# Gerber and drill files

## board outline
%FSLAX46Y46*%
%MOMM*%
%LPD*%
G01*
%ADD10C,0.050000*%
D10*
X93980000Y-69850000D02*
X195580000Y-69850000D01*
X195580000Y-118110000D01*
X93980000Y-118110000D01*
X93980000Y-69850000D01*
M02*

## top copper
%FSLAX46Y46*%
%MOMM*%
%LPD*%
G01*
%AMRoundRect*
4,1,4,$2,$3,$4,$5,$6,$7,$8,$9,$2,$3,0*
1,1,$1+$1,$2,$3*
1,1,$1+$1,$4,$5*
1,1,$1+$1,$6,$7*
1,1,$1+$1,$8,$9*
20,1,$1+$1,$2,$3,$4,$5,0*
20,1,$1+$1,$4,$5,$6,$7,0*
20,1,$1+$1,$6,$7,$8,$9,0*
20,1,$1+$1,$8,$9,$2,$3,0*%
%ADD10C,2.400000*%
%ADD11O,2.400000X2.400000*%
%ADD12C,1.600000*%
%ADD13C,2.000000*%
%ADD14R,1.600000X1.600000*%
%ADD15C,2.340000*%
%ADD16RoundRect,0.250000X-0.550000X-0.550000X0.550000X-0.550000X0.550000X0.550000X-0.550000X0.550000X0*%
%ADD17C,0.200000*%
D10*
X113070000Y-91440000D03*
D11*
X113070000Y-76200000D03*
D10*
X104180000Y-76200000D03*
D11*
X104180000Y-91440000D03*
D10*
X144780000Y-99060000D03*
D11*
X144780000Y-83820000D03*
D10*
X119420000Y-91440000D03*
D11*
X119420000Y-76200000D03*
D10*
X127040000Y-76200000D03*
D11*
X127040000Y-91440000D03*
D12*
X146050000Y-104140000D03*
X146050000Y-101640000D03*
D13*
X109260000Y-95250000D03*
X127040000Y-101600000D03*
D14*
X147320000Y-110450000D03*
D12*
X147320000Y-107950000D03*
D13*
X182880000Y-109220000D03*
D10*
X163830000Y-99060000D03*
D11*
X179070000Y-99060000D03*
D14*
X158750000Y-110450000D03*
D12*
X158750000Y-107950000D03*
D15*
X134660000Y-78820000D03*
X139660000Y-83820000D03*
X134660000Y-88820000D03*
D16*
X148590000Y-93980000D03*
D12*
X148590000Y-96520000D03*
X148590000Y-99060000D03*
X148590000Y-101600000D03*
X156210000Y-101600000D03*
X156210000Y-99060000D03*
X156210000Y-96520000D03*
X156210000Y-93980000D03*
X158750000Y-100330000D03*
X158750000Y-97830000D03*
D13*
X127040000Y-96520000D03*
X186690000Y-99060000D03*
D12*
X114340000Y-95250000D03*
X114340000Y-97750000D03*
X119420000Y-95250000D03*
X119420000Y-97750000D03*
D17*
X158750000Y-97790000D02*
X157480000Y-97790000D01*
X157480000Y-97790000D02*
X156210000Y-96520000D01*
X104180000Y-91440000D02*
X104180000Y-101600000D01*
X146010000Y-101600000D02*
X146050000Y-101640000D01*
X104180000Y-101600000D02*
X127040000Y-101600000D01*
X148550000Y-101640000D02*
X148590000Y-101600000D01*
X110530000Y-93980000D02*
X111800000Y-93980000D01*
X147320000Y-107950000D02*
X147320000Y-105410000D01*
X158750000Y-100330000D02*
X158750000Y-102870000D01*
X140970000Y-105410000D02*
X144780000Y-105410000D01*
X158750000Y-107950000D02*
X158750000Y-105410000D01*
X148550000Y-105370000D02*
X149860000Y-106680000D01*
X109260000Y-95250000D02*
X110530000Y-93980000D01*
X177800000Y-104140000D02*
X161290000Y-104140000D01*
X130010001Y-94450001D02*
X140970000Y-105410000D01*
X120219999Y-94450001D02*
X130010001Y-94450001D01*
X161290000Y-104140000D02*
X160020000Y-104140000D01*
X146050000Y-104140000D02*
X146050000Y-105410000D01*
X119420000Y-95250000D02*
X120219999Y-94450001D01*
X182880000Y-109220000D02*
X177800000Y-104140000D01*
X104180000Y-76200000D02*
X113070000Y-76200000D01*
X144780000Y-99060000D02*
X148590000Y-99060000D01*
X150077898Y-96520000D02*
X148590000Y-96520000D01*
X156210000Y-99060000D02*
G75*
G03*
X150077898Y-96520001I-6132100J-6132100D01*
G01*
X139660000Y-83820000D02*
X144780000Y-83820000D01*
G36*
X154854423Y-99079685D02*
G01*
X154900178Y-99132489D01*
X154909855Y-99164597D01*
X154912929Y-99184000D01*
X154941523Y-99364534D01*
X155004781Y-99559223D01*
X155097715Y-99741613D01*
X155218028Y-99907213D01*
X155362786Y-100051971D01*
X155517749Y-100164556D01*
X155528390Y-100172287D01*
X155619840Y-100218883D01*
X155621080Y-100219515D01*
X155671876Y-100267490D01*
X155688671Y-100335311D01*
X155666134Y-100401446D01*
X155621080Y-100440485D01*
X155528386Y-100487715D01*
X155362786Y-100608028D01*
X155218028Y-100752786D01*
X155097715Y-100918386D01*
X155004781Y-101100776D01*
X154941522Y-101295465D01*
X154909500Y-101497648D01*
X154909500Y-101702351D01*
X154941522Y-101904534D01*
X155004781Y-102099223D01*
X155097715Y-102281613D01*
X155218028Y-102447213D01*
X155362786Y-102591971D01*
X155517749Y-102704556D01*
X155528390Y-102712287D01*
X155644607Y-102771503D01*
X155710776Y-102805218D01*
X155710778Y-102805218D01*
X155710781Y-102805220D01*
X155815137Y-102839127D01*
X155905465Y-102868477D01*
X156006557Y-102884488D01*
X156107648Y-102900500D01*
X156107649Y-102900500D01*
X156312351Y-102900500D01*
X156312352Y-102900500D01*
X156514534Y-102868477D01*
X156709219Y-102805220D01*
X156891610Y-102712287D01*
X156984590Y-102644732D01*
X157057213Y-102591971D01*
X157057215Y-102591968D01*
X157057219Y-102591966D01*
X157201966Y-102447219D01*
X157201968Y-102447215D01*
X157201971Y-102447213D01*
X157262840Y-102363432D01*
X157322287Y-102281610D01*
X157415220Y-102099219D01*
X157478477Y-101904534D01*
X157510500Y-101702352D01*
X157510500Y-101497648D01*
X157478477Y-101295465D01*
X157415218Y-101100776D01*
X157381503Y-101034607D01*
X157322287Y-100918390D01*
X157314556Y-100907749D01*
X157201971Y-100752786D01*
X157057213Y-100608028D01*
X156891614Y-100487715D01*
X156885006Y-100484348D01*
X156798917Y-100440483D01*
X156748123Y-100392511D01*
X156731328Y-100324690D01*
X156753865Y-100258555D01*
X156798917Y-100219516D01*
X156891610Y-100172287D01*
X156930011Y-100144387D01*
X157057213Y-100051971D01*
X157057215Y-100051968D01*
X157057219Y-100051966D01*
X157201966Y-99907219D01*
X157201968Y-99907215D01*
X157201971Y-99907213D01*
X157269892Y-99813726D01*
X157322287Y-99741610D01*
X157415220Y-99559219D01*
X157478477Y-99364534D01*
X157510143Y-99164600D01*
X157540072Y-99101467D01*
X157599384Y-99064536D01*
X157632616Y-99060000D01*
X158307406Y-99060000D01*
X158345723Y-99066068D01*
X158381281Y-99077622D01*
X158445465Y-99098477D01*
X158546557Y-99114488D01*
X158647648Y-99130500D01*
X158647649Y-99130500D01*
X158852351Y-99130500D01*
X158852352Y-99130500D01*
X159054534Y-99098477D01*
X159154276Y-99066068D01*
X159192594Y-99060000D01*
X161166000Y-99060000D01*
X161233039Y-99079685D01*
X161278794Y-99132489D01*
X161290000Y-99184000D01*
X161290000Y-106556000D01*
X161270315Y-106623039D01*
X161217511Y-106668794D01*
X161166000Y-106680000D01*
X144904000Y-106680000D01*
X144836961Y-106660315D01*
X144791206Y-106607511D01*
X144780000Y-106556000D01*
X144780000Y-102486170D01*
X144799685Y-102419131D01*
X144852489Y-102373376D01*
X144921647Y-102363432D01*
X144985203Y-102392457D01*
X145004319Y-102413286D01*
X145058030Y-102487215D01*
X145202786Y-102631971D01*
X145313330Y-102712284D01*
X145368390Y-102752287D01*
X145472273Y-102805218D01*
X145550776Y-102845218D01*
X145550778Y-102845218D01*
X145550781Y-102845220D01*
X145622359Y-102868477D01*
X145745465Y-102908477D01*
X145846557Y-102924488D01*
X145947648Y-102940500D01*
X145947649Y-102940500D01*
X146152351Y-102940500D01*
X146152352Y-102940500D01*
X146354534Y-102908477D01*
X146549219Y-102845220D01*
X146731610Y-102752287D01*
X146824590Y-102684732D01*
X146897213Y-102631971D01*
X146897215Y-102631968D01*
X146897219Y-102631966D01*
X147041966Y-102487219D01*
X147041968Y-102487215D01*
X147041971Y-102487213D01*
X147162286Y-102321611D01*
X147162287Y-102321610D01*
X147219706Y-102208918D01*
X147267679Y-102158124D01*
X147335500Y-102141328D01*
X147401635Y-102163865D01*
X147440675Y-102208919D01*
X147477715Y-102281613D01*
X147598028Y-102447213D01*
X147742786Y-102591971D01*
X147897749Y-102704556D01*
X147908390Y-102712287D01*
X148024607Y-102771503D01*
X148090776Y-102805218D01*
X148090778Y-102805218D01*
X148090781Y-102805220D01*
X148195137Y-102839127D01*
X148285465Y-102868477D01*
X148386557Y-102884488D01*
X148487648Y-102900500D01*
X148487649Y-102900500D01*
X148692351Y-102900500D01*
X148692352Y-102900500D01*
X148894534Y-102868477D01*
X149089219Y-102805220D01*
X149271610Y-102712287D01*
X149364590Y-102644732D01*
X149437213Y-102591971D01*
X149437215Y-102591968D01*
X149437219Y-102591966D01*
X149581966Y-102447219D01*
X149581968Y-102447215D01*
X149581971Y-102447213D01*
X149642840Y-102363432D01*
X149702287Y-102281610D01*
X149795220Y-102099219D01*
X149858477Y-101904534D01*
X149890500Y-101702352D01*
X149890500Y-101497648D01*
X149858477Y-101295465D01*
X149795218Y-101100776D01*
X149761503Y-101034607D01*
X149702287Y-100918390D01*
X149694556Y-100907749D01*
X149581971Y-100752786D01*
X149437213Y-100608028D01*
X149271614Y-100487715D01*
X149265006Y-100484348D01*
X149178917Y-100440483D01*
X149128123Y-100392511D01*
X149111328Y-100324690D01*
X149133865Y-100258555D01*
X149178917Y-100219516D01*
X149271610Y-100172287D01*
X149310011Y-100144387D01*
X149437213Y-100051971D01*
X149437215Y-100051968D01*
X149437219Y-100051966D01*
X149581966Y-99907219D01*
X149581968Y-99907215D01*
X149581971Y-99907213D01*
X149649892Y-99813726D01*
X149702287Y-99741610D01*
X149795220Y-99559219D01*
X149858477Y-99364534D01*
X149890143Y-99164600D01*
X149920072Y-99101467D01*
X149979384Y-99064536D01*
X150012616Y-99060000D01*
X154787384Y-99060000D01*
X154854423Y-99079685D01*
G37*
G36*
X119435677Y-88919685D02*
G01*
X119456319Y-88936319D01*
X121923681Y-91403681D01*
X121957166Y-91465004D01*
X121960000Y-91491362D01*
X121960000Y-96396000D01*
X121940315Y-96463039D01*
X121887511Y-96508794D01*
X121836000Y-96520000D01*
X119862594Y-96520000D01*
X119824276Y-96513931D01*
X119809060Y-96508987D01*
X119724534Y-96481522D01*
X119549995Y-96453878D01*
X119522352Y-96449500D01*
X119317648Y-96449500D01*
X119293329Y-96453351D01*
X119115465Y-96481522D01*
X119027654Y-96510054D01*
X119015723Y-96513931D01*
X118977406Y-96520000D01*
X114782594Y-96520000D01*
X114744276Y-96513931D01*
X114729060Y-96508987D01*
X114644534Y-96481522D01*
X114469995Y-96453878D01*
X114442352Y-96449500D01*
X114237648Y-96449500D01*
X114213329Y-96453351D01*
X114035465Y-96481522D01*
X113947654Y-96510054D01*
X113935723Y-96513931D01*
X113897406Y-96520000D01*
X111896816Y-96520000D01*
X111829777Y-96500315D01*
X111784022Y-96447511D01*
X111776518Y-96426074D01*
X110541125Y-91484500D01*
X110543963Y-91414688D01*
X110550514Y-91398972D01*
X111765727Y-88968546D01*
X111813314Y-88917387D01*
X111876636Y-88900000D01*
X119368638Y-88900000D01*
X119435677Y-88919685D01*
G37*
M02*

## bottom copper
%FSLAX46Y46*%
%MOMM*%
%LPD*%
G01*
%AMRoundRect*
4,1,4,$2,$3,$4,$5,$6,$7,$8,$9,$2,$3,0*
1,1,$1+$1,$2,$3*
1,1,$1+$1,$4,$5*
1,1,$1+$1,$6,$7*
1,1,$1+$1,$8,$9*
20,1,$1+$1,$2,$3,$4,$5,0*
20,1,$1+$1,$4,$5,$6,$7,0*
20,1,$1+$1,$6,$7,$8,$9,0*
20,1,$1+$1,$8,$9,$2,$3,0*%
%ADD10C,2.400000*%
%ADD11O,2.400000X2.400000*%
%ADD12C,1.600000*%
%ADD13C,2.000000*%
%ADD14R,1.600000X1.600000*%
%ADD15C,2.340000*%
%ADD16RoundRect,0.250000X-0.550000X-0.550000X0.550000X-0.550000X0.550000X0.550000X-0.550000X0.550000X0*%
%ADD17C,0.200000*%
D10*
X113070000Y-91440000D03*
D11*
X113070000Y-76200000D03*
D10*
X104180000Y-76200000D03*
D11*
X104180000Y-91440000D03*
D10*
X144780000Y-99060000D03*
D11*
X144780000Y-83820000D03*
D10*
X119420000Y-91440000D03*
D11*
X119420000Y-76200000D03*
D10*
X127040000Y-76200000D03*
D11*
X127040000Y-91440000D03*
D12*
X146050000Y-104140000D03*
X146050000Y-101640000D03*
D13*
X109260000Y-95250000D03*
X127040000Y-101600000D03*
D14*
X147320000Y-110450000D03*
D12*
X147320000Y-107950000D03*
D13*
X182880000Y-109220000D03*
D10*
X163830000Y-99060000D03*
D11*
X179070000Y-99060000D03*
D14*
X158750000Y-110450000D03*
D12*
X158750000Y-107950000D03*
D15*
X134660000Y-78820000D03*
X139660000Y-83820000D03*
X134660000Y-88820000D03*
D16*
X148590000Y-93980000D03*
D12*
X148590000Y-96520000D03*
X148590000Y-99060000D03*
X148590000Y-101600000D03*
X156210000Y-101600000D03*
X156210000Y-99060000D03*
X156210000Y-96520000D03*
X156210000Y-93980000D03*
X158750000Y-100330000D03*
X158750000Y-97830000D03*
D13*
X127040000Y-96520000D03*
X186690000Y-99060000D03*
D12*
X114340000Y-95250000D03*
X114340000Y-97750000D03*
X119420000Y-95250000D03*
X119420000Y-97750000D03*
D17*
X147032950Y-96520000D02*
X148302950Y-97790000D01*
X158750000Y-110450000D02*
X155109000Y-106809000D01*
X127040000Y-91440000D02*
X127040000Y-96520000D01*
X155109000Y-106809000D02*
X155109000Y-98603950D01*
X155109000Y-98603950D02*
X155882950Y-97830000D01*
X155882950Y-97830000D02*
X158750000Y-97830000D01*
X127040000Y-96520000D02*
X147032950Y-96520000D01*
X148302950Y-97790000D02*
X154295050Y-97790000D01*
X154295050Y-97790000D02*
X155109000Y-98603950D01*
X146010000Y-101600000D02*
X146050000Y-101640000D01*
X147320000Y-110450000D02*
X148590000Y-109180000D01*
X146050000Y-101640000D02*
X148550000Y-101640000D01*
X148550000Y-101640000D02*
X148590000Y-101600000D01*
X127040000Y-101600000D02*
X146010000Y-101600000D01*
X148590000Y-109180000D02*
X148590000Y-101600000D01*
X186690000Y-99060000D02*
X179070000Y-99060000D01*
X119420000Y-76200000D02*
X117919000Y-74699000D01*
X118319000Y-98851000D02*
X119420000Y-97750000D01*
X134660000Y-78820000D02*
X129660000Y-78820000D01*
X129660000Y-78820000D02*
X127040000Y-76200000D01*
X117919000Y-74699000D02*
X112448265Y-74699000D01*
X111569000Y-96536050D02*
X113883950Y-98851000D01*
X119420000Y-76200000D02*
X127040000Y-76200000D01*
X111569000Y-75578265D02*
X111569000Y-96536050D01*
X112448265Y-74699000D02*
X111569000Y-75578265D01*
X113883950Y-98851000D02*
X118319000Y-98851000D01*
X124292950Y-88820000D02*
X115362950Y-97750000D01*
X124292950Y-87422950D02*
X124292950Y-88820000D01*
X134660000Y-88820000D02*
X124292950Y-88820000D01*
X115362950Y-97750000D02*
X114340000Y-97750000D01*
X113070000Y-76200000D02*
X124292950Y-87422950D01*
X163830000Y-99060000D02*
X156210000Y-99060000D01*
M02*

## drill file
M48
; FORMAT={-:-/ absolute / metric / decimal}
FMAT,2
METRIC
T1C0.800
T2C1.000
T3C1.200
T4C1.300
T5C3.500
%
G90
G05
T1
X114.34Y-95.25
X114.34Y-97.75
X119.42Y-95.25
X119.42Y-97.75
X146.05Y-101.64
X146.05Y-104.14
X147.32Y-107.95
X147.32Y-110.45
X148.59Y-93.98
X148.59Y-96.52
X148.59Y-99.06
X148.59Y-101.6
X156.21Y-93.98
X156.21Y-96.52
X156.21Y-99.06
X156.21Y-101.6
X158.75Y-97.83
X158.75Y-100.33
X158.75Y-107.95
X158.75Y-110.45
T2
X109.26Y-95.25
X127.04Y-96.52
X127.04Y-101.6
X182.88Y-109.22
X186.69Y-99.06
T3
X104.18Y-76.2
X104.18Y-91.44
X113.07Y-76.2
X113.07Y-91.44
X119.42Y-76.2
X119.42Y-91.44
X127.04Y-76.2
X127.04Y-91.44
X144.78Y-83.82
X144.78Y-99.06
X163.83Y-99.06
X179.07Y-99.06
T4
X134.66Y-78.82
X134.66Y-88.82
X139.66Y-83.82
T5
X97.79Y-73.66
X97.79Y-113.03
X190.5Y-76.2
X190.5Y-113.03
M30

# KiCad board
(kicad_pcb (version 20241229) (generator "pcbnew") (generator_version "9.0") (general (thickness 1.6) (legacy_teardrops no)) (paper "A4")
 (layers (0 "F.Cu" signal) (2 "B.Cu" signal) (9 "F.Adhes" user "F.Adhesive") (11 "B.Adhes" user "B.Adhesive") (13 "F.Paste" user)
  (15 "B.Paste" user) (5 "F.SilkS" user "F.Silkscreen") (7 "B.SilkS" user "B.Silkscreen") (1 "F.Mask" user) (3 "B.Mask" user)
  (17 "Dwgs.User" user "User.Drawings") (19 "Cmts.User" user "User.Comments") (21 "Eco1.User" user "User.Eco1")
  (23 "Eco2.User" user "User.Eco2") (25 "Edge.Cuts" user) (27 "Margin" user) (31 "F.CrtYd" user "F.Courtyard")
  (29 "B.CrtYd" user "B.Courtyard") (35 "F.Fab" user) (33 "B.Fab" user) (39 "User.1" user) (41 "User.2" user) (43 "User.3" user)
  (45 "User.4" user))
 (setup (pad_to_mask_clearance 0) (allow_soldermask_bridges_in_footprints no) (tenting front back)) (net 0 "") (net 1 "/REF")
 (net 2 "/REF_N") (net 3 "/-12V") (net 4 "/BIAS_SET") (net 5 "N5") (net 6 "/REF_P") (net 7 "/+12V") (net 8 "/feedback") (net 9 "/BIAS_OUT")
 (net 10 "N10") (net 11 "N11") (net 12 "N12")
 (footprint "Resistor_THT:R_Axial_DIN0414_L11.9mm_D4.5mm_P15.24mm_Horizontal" (layer "F.Cu") (at 113.07 91.44 90)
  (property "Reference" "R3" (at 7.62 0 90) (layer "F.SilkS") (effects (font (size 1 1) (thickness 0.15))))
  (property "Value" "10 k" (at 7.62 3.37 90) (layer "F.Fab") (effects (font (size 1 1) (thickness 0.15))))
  (pad "1" thru_hole circle (at 0 0 90) (size 2.4 2.4) (drill 1.2) (layers "*.Cu" "*.Mask") (remove_unused_layers no) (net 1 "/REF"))
  (pad "2" thru_hole oval (at 15.24 0 90) (size 2.4 2.4) (drill 1.2) (layers "*.Cu" "*.Mask") (remove_unused_layers no) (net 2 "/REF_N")))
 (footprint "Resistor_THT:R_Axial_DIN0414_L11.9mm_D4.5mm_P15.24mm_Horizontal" (layer "F.Cu") (at 104.18 76.2 -90)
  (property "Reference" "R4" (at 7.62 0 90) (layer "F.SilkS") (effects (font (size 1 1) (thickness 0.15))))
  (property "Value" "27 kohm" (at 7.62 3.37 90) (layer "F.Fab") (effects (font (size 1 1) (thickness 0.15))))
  (pad "1" thru_hole circle (at 0 0 270) (size 2.4 2.4) (drill 1.2) (layers "*.Cu" "*.Mask") (remove_unused_layers no) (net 2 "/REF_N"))
  (pad "2" thru_hole oval (at 15.24 0 270) (size 2.4 2.4) (drill 1.2) (layers "*.Cu" "*.Mask") (remove_unused_layers no) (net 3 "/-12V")))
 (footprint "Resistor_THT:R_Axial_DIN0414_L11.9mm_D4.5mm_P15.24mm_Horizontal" (layer "F.Cu") (at 144.78 99.06 90)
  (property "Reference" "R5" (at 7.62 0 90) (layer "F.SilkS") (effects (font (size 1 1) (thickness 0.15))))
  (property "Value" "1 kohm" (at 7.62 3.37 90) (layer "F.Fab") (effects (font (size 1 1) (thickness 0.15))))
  (pad "1" thru_hole circle (at 0 0 90) (size 2.4 2.4) (drill 1.2) (layers "*.Cu" "*.Mask") (remove_unused_layers no) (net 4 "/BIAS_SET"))
  (pad "2" thru_hole oval (at 15.24 0 90) (size 2.4 2.4) (drill 1.2) (layers "*.Cu" "*.Mask") (remove_unused_layers no) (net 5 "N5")))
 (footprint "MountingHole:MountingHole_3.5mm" (layer "F.Cu") (at 190.5 113.03)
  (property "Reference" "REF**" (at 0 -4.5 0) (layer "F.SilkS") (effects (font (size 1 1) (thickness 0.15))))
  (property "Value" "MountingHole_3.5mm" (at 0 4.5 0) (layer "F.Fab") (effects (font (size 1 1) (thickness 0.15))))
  (pad "" np_thru_hole circle (at 0 0) (size 3.5 3.5) (drill 3.5) (layers "*.Cu" "*.Mask")))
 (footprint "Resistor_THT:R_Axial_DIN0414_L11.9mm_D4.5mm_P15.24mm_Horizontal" (layer "F.Cu") (at 119.42 91.44 90)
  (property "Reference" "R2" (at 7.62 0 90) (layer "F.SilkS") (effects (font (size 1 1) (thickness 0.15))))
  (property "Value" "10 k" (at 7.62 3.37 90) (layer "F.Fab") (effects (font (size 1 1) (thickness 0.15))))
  (pad "1" thru_hole circle (at 0 0 90) (size 2.4 2.4) (drill 1.2) (layers "*.Cu" "*.Mask") (remove_unused_layers no) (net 1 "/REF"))
  (pad "2" thru_hole oval (at 15.24 0 90) (size 2.4 2.4) (drill 1.2) (layers "*.Cu" "*.Mask") (remove_unused_layers no) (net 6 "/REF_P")))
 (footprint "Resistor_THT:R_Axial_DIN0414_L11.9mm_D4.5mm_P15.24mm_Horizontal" (layer "F.Cu") (at 127.04 76.2 -90)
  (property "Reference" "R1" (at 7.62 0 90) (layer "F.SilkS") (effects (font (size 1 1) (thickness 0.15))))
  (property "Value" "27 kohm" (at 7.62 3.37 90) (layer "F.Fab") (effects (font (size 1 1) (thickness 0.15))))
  (pad "1" thru_hole circle (at 0 0 270) (size 2.4 2.4) (drill 1.2) (layers "*.Cu" "*.Mask") (remove_unused_layers no) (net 6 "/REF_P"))
  (pad "2" thru_hole oval (at 15.24 0 270) (size 2.4 2.4) (drill 1.2) (layers "*.Cu" "*.Mask") (remove_unused_layers no) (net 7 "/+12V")))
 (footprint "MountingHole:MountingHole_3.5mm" (layer "F.Cu") (at 190.5 76.2)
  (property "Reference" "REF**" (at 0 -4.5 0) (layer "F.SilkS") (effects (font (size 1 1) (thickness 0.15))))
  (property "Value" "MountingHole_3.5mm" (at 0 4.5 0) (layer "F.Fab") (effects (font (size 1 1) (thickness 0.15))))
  (pad "" np_thru_hole circle (at 0 0) (size 3.5 3.5) (drill 3.5) (layers "*.Cu" "*.Mask")))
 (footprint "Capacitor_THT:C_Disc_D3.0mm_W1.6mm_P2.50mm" (layer "F.Cu") (at 146.05 104.14 90)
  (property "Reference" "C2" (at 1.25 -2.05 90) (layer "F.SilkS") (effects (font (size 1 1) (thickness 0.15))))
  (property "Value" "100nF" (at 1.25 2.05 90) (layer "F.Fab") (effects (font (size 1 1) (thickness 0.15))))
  (pad "1" thru_hole circle (at 0 0 90) (size 1.6 1.6) (drill 0.8) (layers "*.Cu" "*.Mask") (remove_unused_layers no) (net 1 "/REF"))
  (pad "2" thru_hole circle (at 2.5 0 90) (size 1.6 1.6) (drill 0.8) (layers "*.Cu" "*.Mask") (remove_unused_layers no) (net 3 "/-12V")))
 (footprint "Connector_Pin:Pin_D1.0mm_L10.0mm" (layer "F.Cu") (at 109.26 95.25)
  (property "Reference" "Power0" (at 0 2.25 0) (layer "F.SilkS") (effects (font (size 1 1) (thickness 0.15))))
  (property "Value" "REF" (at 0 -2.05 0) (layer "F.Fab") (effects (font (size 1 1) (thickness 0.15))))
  (pad "1" thru_hole circle (at 0 0) (size 2 2) (drill 1) (layers "*.Cu" "*.Mask") (remove_unused_layers no) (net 1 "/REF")))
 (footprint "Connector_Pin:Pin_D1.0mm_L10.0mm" (layer "F.Cu") (at 127.04 101.6)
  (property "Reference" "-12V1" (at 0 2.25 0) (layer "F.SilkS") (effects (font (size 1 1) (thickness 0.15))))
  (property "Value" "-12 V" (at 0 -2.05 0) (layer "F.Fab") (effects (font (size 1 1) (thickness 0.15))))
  (pad "1" thru_hole circle (at 0 0) (size 2 2) (drill 1) (layers "*.Cu" "*.Mask") (remove_unused_layers no) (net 3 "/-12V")))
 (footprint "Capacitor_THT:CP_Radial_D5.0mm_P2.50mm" (layer "F.Cu") (at 147.32 110.45 90)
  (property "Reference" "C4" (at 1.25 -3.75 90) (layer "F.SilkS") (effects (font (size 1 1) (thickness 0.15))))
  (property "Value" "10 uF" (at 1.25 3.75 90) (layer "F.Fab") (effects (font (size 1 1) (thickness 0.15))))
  (pad "1" thru_hole rect (at 0 0 90) (size 1.6 1.6) (drill 0.8) (layers "*.Cu" "*.Mask") (remove_unused_layers no) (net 3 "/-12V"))
  (pad "2" thru_hole circle (at 2.5 0 90) (size 1.6 1.6) (drill 0.8) (layers "*.Cu" "*.Mask") (remove_unused_layers no) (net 1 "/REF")))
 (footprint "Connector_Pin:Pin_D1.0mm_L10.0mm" (layer "F.Cu") (at 182.88 109.22)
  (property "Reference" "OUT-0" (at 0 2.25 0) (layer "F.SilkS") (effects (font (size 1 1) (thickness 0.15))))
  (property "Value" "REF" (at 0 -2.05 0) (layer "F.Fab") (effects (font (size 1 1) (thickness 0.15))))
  (pad "1" thru_hole circle (at 0 0) (size 2 2) (drill 1) (layers "*.Cu" "*.Mask") (remove_unused_layers no) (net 1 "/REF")))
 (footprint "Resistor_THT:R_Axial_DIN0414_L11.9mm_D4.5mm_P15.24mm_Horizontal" (layer "F.Cu") (at 163.83 99.06)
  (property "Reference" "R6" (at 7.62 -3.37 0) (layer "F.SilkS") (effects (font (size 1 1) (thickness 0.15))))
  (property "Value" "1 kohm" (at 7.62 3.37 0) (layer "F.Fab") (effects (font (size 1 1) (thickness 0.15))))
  (pad "1" thru_hole circle (at 0 0) (size 2.4 2.4) (drill 1.2) (layers "*.Cu" "*.Mask") (remove_unused_layers no) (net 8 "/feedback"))
  (pad "2" thru_hole oval (at 15.24 0) (size 2.4 2.4) (drill 1.2) (layers "*.Cu" "*.Mask") (remove_unused_layers no) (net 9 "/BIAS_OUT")))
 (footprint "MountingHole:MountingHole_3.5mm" (layer "F.Cu") (at 97.79 73.66)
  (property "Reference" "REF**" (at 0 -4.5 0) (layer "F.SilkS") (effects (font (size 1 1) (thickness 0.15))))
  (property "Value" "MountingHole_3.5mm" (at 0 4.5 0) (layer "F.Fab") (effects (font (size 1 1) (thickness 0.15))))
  (pad "" np_thru_hole circle (at 0 0) (size 3.5 3.5) (drill 3.5) (layers "*.Cu" "*.Mask")))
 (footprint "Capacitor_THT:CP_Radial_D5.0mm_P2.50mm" (layer "F.Cu") (at 158.75 110.45 90)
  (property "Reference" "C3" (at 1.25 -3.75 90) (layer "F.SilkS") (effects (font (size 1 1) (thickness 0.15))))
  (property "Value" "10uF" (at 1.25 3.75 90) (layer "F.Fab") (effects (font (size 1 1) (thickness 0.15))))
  (pad "1" thru_hole rect (at 0 0 90) (size 1.6 1.6) (drill 0.8) (layers "*.Cu" "*.Mask") (remove_unused_layers no) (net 7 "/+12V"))
  (pad "2" thru_hole circle (at 2.5 0 90) (size 1.6 1.6) (drill 0.8) (layers "*.Cu" "*.Mask") (remove_unused_layers no) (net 1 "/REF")))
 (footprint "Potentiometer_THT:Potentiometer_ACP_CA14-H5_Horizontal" (layer "F.Cu") (at 134.66 78.82)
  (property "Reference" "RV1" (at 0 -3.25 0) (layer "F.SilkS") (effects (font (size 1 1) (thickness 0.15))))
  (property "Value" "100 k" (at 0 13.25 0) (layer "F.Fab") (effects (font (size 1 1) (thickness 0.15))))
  (pad "1" thru_hole circle (at 0 0) (size 2.34 2.34) (drill 1.3) (layers "*.Cu" "*.Mask") (remove_unused_layers no) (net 6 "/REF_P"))
  (pad "2" thru_hole circle (at 5 5) (size 2.34 2.34) (drill 1.3) (layers "*.Cu" "*.Mask") (remove_unused_layers no) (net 5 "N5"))
  (pad "3" thru_hole circle (at 0 10) (size 2.34 2.34) (drill 1.3) (layers "*.Cu" "*.Mask") (remove_unused_layers no) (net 2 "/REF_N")))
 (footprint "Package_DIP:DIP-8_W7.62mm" (layer "F.Cu") (at 148.59 93.98)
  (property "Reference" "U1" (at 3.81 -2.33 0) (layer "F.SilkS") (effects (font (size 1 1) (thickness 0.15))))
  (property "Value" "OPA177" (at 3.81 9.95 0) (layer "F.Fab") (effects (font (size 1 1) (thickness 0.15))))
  (pad "1" thru_hole roundrect (at 0 0) (size 1.6 1.6) (drill 0.8) (layers "*.Cu" "*.Mask") (remove_unused_layers no)
   (roundrect_rratio 0.15625) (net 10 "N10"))
  (pad "2" thru_hole circle (at 0 2.54) (size 1.6 1.6) (drill 0.8) (layers "*.Cu" "*.Mask") (remove_unused_layers no) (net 8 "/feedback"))
  (pad "3" thru_hole circle (at 0 5.08) (size 1.6 1.6) (drill 0.8) (layers "*.Cu" "*.Mask") (remove_unused_layers no) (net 4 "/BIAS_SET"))
  (pad "4" thru_hole circle (at 0 7.62) (size 1.6 1.6) (drill 0.8) (layers "*.Cu" "*.Mask") (remove_unused_layers no) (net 3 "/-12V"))
  (pad "5" thru_hole circle (at 7.62 7.62) (size 1.6 1.6) (drill 0.8) (layers "*.Cu" "*.Mask") (remove_unused_layers no) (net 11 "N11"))
  (pad "6" thru_hole circle (at 7.62 5.08) (size 1.6 1.6) (drill 0.8) (layers "*.Cu" "*.Mask") (remove_unused_layers no) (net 8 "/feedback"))
  (pad "7" thru_hole circle (at 7.62 2.54) (size 1.6 1.6) (drill 0.8) (layers "*.Cu" "*.Mask") (remove_unused_layers no) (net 7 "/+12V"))
  (pad "8" thru_hole circle (at 7.62 0) (size 1.6 1.6) (drill 0.8) (layers "*.Cu" "*.Mask") (remove_unused_layers no) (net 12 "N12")))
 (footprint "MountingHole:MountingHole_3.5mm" (layer "F.Cu") (at 97.79 113.03)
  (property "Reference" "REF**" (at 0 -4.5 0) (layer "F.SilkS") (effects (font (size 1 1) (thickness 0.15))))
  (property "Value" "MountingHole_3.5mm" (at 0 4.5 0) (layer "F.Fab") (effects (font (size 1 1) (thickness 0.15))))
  (pad "" np_thru_hole circle (at 0 0) (size 3.5 3.5) (drill 3.5) (layers "*.Cu" "*.Mask")))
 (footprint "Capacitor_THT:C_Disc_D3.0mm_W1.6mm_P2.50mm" (layer "F.Cu") (at 158.75 100.33 90)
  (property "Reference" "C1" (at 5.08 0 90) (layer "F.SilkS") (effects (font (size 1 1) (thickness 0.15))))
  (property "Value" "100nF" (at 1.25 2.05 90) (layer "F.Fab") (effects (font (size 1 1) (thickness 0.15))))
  (pad "1" thru_hole circle (at 0 0 90) (size 1.6 1.6) (drill 0.8) (layers "*.Cu" "*.Mask") (remove_unused_layers no) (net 1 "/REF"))
  (pad "2" thru_hole circle (at 2.5 0 90) (size 1.6 1.6) (drill 0.8) (layers "*.Cu" "*.Mask") (remove_unused_layers no) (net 7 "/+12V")))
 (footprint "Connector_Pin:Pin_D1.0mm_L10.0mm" (layer "F.Cu") (at 127.04 96.52)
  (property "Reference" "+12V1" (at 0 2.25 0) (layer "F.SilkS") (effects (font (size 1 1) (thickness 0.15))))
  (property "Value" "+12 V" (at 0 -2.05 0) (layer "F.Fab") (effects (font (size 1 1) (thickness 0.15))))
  (pad "1" thru_hole circle (at 0 0) (size 2 2) (drill 1) (layers "*.Cu" "*.Mask") (remove_unused_layers no) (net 7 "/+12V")))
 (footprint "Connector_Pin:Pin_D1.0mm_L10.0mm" (layer "F.Cu") (at 186.69 99.06)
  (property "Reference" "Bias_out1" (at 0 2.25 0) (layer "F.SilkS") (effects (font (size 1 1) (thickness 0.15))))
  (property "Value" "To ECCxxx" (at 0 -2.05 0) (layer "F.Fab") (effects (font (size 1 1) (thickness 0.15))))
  (pad "1" thru_hole circle (at 0 0) (size 2 2) (drill 1) (layers "*.Cu" "*.Mask") (remove_unused_layers no) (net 9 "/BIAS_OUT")))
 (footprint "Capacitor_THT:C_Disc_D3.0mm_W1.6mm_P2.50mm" (layer "F.Cu") (at 114.34 95.25 -90)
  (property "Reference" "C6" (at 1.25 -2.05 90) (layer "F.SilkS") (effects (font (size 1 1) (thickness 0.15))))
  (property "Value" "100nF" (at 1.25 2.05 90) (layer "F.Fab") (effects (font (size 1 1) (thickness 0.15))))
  (pad "1" thru_hole circle (at 0 0 270) (size 1.6 1.6) (drill 0.8) (layers "*.Cu" "*.Mask") (remove_unused_layers no) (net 1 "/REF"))
  (pad "2" thru_hole circle (at 2.5 0 270) (size 1.6 1.6) (drill 0.8) (layers "*.Cu" "*.Mask") (remove_unused_layers no) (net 2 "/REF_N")))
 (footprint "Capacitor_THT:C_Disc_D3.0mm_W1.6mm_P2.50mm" (layer "F.Cu") (at 119.42 95.25 -90)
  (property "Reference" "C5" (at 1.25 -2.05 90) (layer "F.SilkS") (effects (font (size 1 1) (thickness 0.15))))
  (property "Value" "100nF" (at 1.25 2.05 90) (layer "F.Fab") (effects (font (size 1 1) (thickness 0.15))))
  (pad "1" thru_hole circle (at 0 0 270) (size 1.6 1.6) (drill 0.8) (layers "*.Cu" "*.Mask") (remove_unused_layers no) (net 1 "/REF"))
  (pad "2" thru_hole circle (at 2.5 0 270) (size 1.6 1.6) (drill 0.8) (layers "*.Cu" "*.Mask") (remove_unused_layers no) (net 6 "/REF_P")))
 (gr_rect (start 93.98 69.85) (end 195.58 118.11) (stroke (width 0.05) (type default)) (fill no) (layer "Edge.Cuts"))
 (segment (start 158.75 97.79) (end 157.48 97.79) (width 0.2) (layer "F.Cu") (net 7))
 (segment (start 157.48 97.79) (end 156.21 96.52) (width 0.2) (layer "F.Cu") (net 7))
 (segment (start 147.03295 96.52) (end 148.30295 97.79) (width 0.2) (layer "B.Cu") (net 7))
 (segment (start 158.75 110.45) (end 155.109 106.809) (width 0.2) (layer "B.Cu") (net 7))
 (segment (start 127.04 91.44) (end 127.04 96.52) (width 0.2) (layer "B.Cu") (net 7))
 (segment (start 155.109 106.809) (end 155.109 98.60395) (width 0.2) (layer "B.Cu") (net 7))
 (segment (start 155.109 98.60395) (end 155.88295 97.83) (width 0.2) (layer "B.Cu") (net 7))
 (segment (start 155.88295 97.83) (end 158.75 97.83) (width 0.2) (layer "B.Cu") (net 7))
 (segment (start 127.04 96.52) (end 147.03295 96.52) (width 0.2) (layer "B.Cu") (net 7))
 (segment (start 148.30295 97.79) (end 154.29505 97.79) (width 0.2) (layer "B.Cu") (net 7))
 (segment (start 154.29505 97.79) (end 155.109 98.60395) (width 0.2) (layer "B.Cu") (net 7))
 (segment (start 104.18 91.44) (end 104.18 101.6) (width 0.2) (layer "F.Cu") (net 3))
 (segment (start 146.01 101.6) (end 146.05 101.64) (width 0.2) (layer "F.Cu") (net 3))
 (segment (start 104.18 101.6) (end 127.04 101.6) (width 0.2) (layer "F.Cu") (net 3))
 (segment (start 148.55 101.64) (end 148.59 101.6) (width 0.2) (layer "F.Cu") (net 3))
 (segment (start 146.01 101.6) (end 146.05 101.64) (width 0.2) (layer "B.Cu") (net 3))
 (segment (start 147.32 110.45) (end 148.59 109.18) (width 0.2) (layer "B.Cu") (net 3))
 (segment (start 146.05 101.64) (end 148.55 101.64) (width 0.2) (layer "B.Cu") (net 3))
 (segment (start 148.55 101.64) (end 148.59 101.6) (width 0.2) (layer "B.Cu") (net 3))
 (segment (start 127.04 101.6) (end 146.01 101.6) (width 0.2) (layer "B.Cu") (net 3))
 (segment (start 148.59 109.18) (end 148.59 101.6) (width 0.2) (layer "B.Cu") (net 3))
 (segment (start 186.69 99.06) (end 179.07 99.06) (width 0.2) (layer "B.Cu") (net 9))
 (segment (start 110.53 93.98) (end 111.8 93.98) (width 0.2) (layer "F.Cu") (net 1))
 (segment (start 147.32 107.95) (end 147.32 105.41) (width 0.2) (layer "F.Cu") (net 1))
 (segment (start 158.75 100.33) (end 158.75 102.87) (width 0.2) (layer "F.Cu") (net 1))
 (segment (start 140.97 105.41) (end 144.78 105.41) (width 0.2) (layer "F.Cu") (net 1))
 (segment (start 158.75 107.95) (end 158.75 105.41) (width 0.2) (layer "F.Cu") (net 1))
 (segment (start 148.55 105.37) (end 149.86 106.68) (width 0.2) (layer "F.Cu") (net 1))
 (segment (start 109.26 95.25) (end 110.53 93.98) (width 0.2) (layer "F.Cu") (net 1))
 (segment (start 177.8 104.14) (end 161.29 104.14) (width 0.2) (layer "F.Cu") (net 1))
 (segment (start 130.010001 94.450001) (end 140.97 105.41) (width 0.2) (layer "F.Cu") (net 1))
 (segment (start 120.219999 94.450001) (end 130.010001 94.450001) (width 0.2) (layer "F.Cu") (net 1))
 (segment (start 161.29 104.14) (end 160.02 104.14) (width 0.2) (layer "F.Cu") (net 1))
 (segment (start 146.05 104.14) (end 146.05 105.41) (width 0.2) (layer "F.Cu") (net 1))
 (segment (start 119.42 95.25) (end 120.219999 94.450001) (width 0.2) (layer "F.Cu") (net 1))
 (segment (start 182.88 109.22) (end 177.8 104.14) (width 0.2) (layer "F.Cu") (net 1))
 (segment (start 119.42 76.2) (end 117.919 74.699) (width 0.2) (layer "B.Cu") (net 6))
 (segment (start 118.319 98.851) (end 119.42 97.75) (width 0.2) (layer "B.Cu") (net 6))
 (segment (start 134.66 78.82) (end 129.66 78.82) (width 0.2) (layer "B.Cu") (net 6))
 (segment (start 129.66 78.82) (end 127.04 76.2) (width 0.2) (layer "B.Cu") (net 6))
 (segment (start 117.919 74.699) (end 112.448265 74.699) (width 0.2) (layer "B.Cu") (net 6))
 (segment (start 111.569 96.53605) (end 113.88395 98.851) (width 0.2) (layer "B.Cu") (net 6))
 (segment (start 119.42 76.2) (end 127.04 76.2) (width 0.2) (layer "B.Cu") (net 6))
 (segment (start 111.569 75.578265) (end 111.569 96.53605) (width 0.2) (layer "B.Cu") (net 6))
 (segment (start 112.448265 74.699) (end 111.569 75.578265) (width 0.2) (layer "B.Cu") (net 6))
 (segment (start 113.88395 98.851) (end 118.319 98.851) (width 0.2) (layer "B.Cu") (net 6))
 (segment (start 104.18 76.2) (end 113.07 76.2) (width 0.2) (layer "F.Cu") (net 2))
 (segment (start 124.29295 88.82) (end 115.36295 97.75) (width 0.2) (layer "B.Cu") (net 2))
 (segment (start 124.29295 87.42295) (end 124.29295 88.82) (width 0.2) (layer "B.Cu") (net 2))
 (segment (start 134.66 88.82) (end 124.29295 88.82) (width 0.2) (layer "B.Cu") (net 2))
 (segment (start 115.36295 97.75) (end 114.34 97.75) (width 0.2) (layer "B.Cu") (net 2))
 (segment (start 113.07 76.2) (end 124.29295 87.42295) (width 0.2) (layer "B.Cu") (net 2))
 (segment (start 144.78 99.06) (end 148.59 99.06) (width 0.2) (layer "F.Cu") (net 4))
 (segment (start 150.077898 96.52) (end 148.59 96.52) (width 0.2) (layer "F.Cu") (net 8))
 (arc (start 156.21 99.06) (mid 153.396568 97.180124) (end 150.077898 96.52) (width 0.2) (layer "F.Cu") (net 8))
 (segment (start 163.83 99.06) (end 156.21 99.06) (width 0.2) (layer "B.Cu") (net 8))
 (segment (start 139.66 83.82) (end 144.78 83.82) (width 0.2) (layer "F.Cu") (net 5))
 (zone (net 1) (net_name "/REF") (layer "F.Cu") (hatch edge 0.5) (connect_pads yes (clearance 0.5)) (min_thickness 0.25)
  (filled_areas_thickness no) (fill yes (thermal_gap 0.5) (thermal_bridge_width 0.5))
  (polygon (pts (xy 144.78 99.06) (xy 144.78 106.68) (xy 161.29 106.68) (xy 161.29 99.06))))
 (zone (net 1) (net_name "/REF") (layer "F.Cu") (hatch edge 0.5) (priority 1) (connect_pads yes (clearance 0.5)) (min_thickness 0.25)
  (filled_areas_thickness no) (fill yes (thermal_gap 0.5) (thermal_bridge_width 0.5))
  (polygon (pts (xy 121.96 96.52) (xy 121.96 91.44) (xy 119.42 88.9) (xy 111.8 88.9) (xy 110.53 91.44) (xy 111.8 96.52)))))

